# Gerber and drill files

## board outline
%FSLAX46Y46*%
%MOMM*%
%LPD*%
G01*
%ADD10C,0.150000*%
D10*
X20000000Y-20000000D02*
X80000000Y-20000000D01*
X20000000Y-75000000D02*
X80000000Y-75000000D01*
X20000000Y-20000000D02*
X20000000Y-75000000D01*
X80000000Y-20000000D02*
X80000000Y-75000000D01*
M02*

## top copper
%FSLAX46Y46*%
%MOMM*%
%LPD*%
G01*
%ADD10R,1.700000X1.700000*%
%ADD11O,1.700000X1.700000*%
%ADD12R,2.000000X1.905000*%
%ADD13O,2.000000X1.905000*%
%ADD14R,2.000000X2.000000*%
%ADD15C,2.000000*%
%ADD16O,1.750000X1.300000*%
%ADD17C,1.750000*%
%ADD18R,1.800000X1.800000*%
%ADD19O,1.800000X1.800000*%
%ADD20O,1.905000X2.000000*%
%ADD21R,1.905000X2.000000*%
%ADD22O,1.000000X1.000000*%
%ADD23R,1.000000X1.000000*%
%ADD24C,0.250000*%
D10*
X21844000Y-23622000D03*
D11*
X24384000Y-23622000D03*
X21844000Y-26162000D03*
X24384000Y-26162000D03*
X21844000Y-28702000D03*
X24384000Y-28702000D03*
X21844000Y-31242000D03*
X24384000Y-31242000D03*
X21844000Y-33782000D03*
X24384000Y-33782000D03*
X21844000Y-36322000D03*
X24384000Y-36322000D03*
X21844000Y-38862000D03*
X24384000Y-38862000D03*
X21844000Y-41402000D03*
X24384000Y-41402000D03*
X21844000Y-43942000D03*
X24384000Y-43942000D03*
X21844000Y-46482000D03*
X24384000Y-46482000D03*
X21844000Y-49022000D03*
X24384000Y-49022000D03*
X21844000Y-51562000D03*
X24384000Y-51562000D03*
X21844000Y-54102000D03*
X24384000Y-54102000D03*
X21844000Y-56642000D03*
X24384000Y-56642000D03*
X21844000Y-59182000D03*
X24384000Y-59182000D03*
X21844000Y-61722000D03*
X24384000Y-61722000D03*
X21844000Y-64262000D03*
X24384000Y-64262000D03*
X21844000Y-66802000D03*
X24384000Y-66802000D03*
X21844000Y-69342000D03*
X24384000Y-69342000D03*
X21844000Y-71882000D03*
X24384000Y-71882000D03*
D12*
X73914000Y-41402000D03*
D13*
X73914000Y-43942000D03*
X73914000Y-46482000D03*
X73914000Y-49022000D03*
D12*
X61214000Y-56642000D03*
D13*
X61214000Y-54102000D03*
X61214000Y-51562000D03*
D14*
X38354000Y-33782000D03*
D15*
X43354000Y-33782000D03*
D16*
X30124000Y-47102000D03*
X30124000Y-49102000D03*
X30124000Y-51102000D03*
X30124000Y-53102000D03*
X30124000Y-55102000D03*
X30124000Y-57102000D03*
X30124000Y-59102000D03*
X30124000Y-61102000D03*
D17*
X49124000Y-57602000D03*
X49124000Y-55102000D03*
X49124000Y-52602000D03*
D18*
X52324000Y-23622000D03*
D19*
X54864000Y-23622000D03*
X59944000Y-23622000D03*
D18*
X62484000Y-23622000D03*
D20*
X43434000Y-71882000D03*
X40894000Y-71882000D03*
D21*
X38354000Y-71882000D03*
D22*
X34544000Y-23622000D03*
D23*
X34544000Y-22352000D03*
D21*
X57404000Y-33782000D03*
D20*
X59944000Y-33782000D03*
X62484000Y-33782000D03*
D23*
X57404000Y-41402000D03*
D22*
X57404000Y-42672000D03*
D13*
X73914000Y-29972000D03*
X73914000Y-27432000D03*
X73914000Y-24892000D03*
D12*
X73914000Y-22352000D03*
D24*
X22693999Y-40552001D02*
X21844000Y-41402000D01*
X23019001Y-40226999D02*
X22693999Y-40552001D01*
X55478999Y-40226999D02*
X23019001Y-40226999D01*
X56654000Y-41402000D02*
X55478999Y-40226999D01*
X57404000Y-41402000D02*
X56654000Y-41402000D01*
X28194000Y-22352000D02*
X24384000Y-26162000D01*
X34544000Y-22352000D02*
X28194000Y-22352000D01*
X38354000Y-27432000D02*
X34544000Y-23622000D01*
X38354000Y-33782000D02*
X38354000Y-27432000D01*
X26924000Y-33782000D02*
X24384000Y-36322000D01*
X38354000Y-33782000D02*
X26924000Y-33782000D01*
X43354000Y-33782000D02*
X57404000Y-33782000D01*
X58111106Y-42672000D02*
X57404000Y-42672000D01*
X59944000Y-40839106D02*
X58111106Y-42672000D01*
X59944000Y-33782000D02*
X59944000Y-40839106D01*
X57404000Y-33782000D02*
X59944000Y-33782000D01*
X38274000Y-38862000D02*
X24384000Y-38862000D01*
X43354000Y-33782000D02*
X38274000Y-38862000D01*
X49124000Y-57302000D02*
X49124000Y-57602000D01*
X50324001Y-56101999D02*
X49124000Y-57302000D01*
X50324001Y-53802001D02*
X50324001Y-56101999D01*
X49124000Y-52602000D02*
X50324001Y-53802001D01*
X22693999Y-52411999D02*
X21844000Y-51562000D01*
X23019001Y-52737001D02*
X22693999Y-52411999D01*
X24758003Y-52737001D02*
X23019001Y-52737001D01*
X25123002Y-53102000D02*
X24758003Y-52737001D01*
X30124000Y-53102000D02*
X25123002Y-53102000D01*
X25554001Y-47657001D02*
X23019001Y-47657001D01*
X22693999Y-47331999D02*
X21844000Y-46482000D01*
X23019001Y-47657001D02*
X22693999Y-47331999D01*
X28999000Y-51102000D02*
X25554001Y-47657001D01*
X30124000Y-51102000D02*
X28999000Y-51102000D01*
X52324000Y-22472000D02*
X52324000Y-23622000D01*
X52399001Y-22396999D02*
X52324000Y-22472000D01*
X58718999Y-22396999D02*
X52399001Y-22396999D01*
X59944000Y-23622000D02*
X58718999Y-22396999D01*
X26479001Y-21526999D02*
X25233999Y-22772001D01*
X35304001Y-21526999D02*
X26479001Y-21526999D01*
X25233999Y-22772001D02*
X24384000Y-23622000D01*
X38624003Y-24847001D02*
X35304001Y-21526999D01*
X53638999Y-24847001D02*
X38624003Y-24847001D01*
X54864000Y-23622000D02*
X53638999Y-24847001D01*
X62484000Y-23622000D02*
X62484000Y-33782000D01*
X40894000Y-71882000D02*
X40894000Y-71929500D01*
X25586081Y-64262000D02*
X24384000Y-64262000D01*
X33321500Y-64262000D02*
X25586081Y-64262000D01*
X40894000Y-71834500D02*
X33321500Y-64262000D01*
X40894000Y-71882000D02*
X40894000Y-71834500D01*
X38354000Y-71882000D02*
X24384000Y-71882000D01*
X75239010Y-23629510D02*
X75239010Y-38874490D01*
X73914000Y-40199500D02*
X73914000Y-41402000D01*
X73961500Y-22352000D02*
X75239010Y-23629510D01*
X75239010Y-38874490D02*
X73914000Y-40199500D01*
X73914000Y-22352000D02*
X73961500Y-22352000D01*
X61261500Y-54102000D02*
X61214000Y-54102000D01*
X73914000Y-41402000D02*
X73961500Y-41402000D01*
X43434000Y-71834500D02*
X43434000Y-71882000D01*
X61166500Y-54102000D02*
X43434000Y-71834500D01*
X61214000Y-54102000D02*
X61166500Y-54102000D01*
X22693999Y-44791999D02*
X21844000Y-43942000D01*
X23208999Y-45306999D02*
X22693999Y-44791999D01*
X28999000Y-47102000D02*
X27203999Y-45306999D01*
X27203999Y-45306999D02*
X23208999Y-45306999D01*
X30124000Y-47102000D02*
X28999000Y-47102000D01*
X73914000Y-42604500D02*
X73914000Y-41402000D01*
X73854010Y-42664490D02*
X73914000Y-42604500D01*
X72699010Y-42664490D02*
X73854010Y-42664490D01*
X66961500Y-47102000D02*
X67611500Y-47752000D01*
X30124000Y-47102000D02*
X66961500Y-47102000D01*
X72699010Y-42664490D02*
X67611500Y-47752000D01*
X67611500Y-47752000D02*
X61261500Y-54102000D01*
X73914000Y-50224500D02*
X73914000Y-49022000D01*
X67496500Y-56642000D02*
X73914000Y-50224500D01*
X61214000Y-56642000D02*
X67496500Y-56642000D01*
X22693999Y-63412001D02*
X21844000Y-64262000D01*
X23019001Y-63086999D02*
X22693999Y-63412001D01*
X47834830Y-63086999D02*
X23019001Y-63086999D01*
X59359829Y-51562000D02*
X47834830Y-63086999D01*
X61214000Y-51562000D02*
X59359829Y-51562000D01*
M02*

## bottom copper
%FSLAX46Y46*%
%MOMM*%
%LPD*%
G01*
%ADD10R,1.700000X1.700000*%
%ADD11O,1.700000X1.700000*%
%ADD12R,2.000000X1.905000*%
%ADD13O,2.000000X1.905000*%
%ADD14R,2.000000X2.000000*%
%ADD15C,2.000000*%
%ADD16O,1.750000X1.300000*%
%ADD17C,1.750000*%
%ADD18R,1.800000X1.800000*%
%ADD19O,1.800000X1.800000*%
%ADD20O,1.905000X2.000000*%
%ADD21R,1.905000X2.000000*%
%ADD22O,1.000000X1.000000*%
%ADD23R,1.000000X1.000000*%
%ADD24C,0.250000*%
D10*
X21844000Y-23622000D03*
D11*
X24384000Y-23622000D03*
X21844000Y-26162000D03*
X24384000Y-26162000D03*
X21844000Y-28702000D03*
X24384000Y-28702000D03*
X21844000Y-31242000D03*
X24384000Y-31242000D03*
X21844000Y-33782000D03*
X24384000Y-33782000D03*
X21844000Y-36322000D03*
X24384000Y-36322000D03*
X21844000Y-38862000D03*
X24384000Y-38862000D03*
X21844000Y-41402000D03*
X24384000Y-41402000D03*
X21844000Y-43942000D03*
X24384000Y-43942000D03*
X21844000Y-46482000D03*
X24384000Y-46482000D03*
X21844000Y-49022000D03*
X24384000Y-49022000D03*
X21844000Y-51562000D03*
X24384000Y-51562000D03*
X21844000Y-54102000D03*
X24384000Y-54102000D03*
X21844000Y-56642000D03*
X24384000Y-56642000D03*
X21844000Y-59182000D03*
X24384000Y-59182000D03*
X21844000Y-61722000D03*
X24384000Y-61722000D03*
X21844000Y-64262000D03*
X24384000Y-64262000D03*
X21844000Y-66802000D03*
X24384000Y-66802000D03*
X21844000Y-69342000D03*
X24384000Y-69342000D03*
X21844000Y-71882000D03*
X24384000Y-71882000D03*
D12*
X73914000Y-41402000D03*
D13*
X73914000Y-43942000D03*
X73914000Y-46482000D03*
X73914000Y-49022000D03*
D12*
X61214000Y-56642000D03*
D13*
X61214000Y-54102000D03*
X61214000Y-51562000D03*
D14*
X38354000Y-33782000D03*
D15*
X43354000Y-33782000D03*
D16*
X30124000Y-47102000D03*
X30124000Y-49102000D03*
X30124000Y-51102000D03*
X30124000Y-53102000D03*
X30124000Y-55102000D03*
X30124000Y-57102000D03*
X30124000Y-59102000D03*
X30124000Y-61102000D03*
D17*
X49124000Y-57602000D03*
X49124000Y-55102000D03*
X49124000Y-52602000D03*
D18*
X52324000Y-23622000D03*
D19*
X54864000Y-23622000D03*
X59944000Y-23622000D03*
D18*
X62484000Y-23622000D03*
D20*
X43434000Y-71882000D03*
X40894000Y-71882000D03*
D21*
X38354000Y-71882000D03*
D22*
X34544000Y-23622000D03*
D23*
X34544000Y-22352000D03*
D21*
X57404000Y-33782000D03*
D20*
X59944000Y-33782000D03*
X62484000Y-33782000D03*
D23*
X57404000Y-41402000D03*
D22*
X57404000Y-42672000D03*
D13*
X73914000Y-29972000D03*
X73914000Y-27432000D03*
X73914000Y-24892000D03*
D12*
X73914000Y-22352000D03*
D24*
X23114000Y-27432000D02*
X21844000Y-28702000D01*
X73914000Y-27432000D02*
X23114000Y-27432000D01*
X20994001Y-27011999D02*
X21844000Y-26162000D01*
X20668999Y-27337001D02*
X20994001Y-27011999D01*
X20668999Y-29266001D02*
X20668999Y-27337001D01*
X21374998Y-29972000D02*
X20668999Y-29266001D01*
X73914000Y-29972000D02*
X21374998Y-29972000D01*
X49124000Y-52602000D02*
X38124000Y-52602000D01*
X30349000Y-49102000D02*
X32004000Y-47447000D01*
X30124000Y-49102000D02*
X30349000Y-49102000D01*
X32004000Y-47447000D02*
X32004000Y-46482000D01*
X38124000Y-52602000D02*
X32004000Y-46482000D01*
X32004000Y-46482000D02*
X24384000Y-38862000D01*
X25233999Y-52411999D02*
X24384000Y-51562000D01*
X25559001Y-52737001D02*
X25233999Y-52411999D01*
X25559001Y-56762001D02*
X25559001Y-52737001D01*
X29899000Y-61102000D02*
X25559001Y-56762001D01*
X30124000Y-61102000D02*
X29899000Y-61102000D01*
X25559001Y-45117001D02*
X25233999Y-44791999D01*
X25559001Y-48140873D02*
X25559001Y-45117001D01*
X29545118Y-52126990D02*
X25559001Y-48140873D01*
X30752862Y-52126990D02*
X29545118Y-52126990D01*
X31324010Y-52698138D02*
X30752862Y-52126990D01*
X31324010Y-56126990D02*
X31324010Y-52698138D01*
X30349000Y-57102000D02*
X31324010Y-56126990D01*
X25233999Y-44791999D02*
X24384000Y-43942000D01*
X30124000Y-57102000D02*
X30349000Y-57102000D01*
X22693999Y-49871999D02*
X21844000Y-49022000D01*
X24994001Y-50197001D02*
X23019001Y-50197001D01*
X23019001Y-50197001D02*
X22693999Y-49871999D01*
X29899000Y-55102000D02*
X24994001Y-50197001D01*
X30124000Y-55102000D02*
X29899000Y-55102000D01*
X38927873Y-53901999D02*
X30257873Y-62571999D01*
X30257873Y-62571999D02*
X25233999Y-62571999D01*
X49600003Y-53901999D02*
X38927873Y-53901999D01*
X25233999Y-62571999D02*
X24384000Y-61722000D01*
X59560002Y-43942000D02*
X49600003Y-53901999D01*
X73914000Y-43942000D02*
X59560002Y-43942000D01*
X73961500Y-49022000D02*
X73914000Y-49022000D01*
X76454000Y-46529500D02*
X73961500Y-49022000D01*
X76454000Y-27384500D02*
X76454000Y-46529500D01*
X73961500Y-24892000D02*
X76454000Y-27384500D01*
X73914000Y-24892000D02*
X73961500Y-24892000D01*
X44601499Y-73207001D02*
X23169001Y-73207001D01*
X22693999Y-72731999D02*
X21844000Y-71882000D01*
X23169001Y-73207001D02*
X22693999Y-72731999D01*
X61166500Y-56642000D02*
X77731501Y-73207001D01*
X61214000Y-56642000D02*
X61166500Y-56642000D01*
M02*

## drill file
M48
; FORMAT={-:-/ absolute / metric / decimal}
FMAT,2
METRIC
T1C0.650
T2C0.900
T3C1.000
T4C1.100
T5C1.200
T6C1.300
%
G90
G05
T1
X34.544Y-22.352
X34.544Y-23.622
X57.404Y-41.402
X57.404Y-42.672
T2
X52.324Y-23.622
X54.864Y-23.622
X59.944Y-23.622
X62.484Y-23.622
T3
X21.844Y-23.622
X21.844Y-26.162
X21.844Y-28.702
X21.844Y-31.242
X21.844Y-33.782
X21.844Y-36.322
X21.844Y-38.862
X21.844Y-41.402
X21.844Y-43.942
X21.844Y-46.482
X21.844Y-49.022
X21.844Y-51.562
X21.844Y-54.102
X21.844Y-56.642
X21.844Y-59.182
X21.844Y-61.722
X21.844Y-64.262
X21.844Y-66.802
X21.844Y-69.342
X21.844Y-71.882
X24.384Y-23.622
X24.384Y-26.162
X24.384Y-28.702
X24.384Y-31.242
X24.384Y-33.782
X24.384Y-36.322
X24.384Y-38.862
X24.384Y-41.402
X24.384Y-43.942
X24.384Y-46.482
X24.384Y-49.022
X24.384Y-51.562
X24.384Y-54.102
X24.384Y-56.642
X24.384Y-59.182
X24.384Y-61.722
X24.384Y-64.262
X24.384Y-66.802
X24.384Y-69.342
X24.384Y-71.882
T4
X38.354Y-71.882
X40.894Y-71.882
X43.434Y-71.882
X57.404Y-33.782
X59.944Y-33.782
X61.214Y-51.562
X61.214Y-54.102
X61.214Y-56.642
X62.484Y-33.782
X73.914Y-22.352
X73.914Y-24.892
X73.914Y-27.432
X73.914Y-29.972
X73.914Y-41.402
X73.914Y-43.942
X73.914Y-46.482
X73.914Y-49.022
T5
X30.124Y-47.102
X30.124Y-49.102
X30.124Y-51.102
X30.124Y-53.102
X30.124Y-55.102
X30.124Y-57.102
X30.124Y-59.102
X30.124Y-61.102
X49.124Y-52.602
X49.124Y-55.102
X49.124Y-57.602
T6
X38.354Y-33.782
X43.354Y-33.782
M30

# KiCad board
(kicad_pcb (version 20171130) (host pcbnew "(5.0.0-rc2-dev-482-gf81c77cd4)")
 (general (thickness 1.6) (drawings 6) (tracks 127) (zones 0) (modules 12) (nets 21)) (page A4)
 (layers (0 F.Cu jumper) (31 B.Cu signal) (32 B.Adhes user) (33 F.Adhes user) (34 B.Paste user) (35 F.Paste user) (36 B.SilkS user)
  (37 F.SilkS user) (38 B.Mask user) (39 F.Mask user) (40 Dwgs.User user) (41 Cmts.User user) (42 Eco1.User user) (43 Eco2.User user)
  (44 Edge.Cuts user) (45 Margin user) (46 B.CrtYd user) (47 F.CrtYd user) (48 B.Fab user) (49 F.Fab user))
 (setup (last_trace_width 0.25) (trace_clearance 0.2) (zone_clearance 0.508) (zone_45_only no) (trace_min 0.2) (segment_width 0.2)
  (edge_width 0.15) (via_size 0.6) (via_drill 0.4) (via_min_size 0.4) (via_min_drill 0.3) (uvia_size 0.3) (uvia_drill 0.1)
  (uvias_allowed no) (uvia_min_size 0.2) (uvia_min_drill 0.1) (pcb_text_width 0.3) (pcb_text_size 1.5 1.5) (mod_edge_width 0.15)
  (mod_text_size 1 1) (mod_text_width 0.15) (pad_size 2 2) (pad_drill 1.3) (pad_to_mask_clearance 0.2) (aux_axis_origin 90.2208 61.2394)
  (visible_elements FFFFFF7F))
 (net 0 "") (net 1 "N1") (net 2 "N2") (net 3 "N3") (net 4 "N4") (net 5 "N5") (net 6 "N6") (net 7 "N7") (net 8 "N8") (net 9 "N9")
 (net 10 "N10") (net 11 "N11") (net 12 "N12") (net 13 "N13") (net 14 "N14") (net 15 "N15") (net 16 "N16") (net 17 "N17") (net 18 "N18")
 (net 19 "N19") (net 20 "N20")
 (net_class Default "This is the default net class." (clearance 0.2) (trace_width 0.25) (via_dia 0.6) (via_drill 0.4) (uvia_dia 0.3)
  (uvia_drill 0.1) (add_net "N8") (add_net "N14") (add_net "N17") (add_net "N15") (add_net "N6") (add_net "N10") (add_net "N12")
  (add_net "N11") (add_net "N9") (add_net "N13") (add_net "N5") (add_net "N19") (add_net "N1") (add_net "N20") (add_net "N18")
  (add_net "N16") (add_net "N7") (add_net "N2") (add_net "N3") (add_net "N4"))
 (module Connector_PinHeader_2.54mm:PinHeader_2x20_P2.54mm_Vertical (layer F.Cu) (at 21.844 23.622)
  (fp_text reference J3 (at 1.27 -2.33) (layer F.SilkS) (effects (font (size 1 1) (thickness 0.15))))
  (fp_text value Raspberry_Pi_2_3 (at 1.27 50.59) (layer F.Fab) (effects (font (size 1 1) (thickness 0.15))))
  (pad 1 thru_hole rect (at 0 0) (size 1.7 1.7) (drill 1) (layers *.Cu *.Mask))
  (pad 2 thru_hole oval (at 2.54 0) (size 1.7 1.7) (drill 1) (layers *.Cu *.Mask) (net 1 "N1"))
  (pad 3 thru_hole oval (at 0 2.54) (size 1.7 1.7) (drill 1) (layers *.Cu *.Mask) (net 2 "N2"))
  (pad 4 thru_hole oval (at 2.54 2.54) (size 1.7 1.7) (drill 1) (layers *.Cu *.Mask) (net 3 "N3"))
  (pad 5 thru_hole oval (at 0 5.08) (size 1.7 1.7) (drill 1) (layers *.Cu *.Mask) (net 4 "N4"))
  (pad 6 thru_hole oval (at 2.54 5.08) (size 1.7 1.7) (drill 1) (layers *.Cu *.Mask))
  (pad 7 thru_hole oval (at 0 7.62) (size 1.7 1.7) (drill 1) (layers *.Cu *.Mask))
  (pad 8 thru_hole oval (at 2.54 7.62) (size 1.7 1.7) (drill 1) (layers *.Cu *.Mask))
  (pad 9 thru_hole oval (at 0 10.16) (size 1.7 1.7) (drill 1) (layers *.Cu *.Mask))
  (pad 10 thru_hole oval (at 2.54 10.16) (size 1.7 1.7) (drill 1) (layers *.Cu *.Mask))
  (pad 11 thru_hole oval (at 0 12.7) (size 1.7 1.7) (drill 1) (layers *.Cu *.Mask))
  (pad 12 thru_hole oval (at 2.54 12.7) (size 1.7 1.7) (drill 1) (layers *.Cu *.Mask) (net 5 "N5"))
  (pad 13 thru_hole oval (at 0 15.24) (size 1.7 1.7) (drill 1) (layers *.Cu *.Mask))
  (pad 14 thru_hole oval (at 2.54 15.24) (size 1.7 1.7) (drill 1) (layers *.Cu *.Mask) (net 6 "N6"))
  (pad 15 thru_hole oval (at 0 17.78) (size 1.7 1.7) (drill 1) (layers *.Cu *.Mask) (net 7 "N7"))
  (pad 16 thru_hole oval (at 2.54 17.78) (size 1.7 1.7) (drill 1) (layers *.Cu *.Mask))
  (pad 17 thru_hole oval (at 0 20.32) (size 1.7 1.7) (drill 1) (layers *.Cu *.Mask) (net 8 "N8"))
  (pad 18 thru_hole oval (at 2.54 20.32) (size 1.7 1.7) (drill 1) (layers *.Cu *.Mask) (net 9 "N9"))
  (pad 19 thru_hole oval (at 0 22.86) (size 1.7 1.7) (drill 1) (layers *.Cu *.Mask) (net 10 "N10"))
  (pad 20 thru_hole oval (at 2.54 22.86) (size 1.7 1.7) (drill 1) (layers *.Cu *.Mask))
  (pad 21 thru_hole oval (at 0 25.4) (size 1.7 1.7) (drill 1) (layers *.Cu *.Mask) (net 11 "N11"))
  (pad 22 thru_hole oval (at 2.54 25.4) (size 1.7 1.7) (drill 1) (layers *.Cu *.Mask))
  (pad 23 thru_hole oval (at 0 27.94) (size 1.7 1.7) (drill 1) (layers *.Cu *.Mask) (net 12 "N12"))
  (pad 24 thru_hole oval (at 2.54 27.94) (size 1.7 1.7) (drill 1) (layers *.Cu *.Mask) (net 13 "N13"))
  (pad 25 thru_hole oval (at 0 30.48) (size 1.7 1.7) (drill 1) (layers *.Cu *.Mask))
  (pad 26 thru_hole oval (at 2.54 30.48) (size 1.7 1.7) (drill 1) (layers *.Cu *.Mask))
  (pad 27 thru_hole oval (at 0 33.02) (size 1.7 1.7) (drill 1) (layers *.Cu *.Mask))
  (pad 28 thru_hole oval (at 2.54 33.02) (size 1.7 1.7) (drill 1) (layers *.Cu *.Mask))
  (pad 29 thru_hole oval (at 0 35.56) (size 1.7 1.7) (drill 1) (layers *.Cu *.Mask))
  (pad 30 thru_hole oval (at 2.54 35.56) (size 1.7 1.7) (drill 1) (layers *.Cu *.Mask))
  (pad 31 thru_hole oval (at 0 38.1) (size 1.7 1.7) (drill 1) (layers *.Cu *.Mask))
  (pad 32 thru_hole oval (at 2.54 38.1) (size 1.7 1.7) (drill 1) (layers *.Cu *.Mask) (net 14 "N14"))
  (pad 33 thru_hole oval (at 0 40.64) (size 1.7 1.7) (drill 1) (layers *.Cu *.Mask) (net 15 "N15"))
  (pad 34 thru_hole oval (at 2.54 40.64) (size 1.7 1.7) (drill 1) (layers *.Cu *.Mask) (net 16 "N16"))
  (pad 35 thru_hole oval (at 0 43.18) (size 1.7 1.7) (drill 1) (layers *.Cu *.Mask))
  (pad 36 thru_hole oval (at 2.54 43.18) (size 1.7 1.7) (drill 1) (layers *.Cu *.Mask))
  (pad 37 thru_hole oval (at 0 45.72) (size 1.7 1.7) (drill 1) (layers *.Cu *.Mask))
  (pad 38 thru_hole oval (at 2.54 45.72) (size 1.7 1.7) (drill 1) (layers *.Cu *.Mask))
  (pad 39 thru_hole oval (at 0 48.26) (size 1.7 1.7) (drill 1) (layers *.Cu *.Mask) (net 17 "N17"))
  (pad 40 thru_hole oval (at 2.54 48.26) (size 1.7 1.7) (drill 1) (layers *.Cu *.Mask) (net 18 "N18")))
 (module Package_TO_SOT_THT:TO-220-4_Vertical (layer F.Cu) (at 73.914 41.402 270)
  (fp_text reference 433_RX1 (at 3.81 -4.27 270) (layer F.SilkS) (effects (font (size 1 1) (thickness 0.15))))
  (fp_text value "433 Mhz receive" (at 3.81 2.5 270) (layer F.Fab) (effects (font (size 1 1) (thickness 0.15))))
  (pad 1 thru_hole rect (at 0 0 270) (size 1.905 2) (drill 1.1) (layers *.Cu *.Mask) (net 8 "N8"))
  (pad 2 thru_hole oval (at 2.54 0 270) (size 1.905 2) (drill 1.1) (layers *.Cu *.Mask) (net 14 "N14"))
  (pad 3 thru_hole oval (at 5.08 0 270) (size 1.905 2) (drill 1.1) (layers *.Cu *.Mask))
  (pad 4 thru_hole oval (at 7.62 0 270) (size 1.905 2) (drill 1.1) (layers *.Cu *.Mask) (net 17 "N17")))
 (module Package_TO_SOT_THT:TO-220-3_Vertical (layer F.Cu) (at 61.214 56.642 90)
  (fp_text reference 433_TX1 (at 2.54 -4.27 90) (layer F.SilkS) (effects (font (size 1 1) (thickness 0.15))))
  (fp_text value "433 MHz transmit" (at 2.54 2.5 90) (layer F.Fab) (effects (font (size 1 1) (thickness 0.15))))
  (pad 1 thru_hole rect (at 0 0 90) (size 1.905 2) (drill 1.1) (layers *.Cu *.Mask) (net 17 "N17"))
  (pad 2 thru_hole oval (at 2.54 0 90) (size 1.905 2) (drill 1.1) (layers *.Cu *.Mask) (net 8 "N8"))
  (pad 3 thru_hole oval (at 5.08 0 90) (size 1.905 2) (drill 1.1) (layers *.Cu *.Mask) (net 15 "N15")))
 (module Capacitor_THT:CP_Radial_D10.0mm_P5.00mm (layer F.Cu) (at 38.354 33.782)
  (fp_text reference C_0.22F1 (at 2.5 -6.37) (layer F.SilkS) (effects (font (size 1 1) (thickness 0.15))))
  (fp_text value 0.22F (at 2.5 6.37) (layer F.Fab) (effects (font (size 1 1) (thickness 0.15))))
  (pad 1 thru_hole rect (at 0 0) (size 2 2) (drill 1.3) (layers *.Cu *.Mask) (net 5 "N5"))
  (pad 2 thru_hole circle (at 5 0) (size 2 2) (drill 1.3) (layers *.Cu *.Mask) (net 6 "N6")))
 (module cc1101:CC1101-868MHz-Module (layer F.Cu) (at 39.624 54.102)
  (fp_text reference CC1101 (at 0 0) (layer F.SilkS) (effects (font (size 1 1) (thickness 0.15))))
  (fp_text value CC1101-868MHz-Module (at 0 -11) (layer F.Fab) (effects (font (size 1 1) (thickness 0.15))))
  (pad 1 thru_hole oval (at -9.5 -7) (size 1.75 1.3) (drill 1.2) (layers *.Cu *.Mask) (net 8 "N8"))
  (pad 2 thru_hole oval (at -9.5 -5) (size 1.75 1.3) (drill 1.2) (layers *.Cu *.Mask) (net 6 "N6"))
  (pad 3 thru_hole oval (at -9.5 -3) (size 1.75 1.3) (drill 1.2) (layers *.Cu *.Mask) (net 10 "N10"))
  (pad 4 thru_hole oval (at -9.5 -1) (size 1.75 1.3) (drill 1.2) (layers *.Cu *.Mask) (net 12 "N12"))
  (pad 5 thru_hole oval (at -9.5 1) (size 1.75 1.3) (drill 1.2) (layers *.Cu *.Mask) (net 11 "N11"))
  (pad 6 thru_hole oval (at -9.5 3) (size 1.75 1.3) (drill 1.2) (layers *.Cu *.Mask) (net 9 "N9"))
  (pad 7 thru_hole oval (at -9.5 5) (size 1.75 1.3) (drill 1.2) (layers *.Cu *.Mask))
  (pad 8 thru_hole oval (at -9.5 7) (size 1.75 1.3) (drill 1.2) (layers *.Cu *.Mask) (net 13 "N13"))
  (pad 9 thru_hole circle (at 9.5 3.5) (size 1.75 1.75) (drill 1.2) (layers *.Cu *.Mask) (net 6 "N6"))
  (pad 10 thru_hole circle (at 9.5 1) (size 1.75 1.75) (drill 1.2) (layers *.Cu *.Mask))
  (pad 11 thru_hole circle (at 9.5 -1.5) (size 1.75 1.75) (drill 1.2) (layers *.Cu *.Mask) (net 6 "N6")))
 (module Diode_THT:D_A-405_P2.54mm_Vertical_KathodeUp (layer F.Cu) (at 52.324 23.622)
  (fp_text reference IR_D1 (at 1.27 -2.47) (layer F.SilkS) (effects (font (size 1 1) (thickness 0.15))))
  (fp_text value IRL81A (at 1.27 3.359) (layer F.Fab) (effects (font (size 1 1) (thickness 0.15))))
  (pad 1 thru_hole rect (at 0 0) (size 1.8 1.8) (drill 0.9) (layers *.Cu *.Mask) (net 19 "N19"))
  (pad 2 thru_hole oval (at 2.54 0) (size 1.8 1.8) (drill 0.9) (layers *.Cu *.Mask) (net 1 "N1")))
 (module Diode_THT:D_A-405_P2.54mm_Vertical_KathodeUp (layer F.Cu) (at 62.484 23.622 180)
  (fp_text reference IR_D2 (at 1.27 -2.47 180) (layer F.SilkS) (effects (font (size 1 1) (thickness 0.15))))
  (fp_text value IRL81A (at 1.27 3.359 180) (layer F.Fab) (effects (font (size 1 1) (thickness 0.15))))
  (pad 2 thru_hole oval (at 2.54 0 180) (size 1.8 1.8) (drill 0.9) (layers *.Cu *.Mask) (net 19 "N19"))
  (pad 1 thru_hole rect (at 0 0 180) (size 1.8 1.8) (drill 0.9) (layers *.Cu *.Mask) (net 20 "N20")))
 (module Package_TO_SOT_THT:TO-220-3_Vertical (layer F.Cu) (at 38.354 71.882)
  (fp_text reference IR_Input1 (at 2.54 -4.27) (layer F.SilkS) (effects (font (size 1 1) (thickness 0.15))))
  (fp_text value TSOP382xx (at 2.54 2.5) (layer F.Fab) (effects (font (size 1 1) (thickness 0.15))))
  (pad 3 thru_hole oval (at 5.08 0) (size 1.905 2) (drill 1.1) (layers *.Cu *.Mask) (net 8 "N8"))
  (pad 2 thru_hole oval (at 2.54 0) (size 1.905 2) (drill 1.1) (layers *.Cu *.Mask) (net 16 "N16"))
  (pad 1 thru_hole rect (at 0 0) (size 1.905 2) (drill 1.1) (layers *.Cu *.Mask) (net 18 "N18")))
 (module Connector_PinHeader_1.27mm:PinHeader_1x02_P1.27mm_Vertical (layer F.Cu) (at 34.544 22.352)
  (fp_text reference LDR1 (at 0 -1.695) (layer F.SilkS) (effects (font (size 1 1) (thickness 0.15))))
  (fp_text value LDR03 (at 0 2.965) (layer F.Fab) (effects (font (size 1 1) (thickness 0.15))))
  (pad 2 thru_hole oval (at 0 1.27) (size 1 1) (drill 0.65) (layers *.Cu *.Mask) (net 5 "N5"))
  (pad 1 thru_hole rect (at 0 0) (size 1 1) (drill 0.65) (layers *.Cu *.Mask) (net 3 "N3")))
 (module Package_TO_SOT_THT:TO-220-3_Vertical (layer F.Cu) (at 57.404 33.782)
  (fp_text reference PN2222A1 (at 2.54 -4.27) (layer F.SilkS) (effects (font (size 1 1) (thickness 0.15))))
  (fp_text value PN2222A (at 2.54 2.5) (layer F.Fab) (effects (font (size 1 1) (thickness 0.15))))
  (pad 1 thru_hole rect (at 0 0) (size 1.905 2) (drill 1.1) (layers *.Cu *.Mask) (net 6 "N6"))
  (pad 2 thru_hole oval (at 2.54 0) (size 1.905 2) (drill 1.1) (layers *.Cu *.Mask) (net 6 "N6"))
  (pad 3 thru_hole oval (at 5.08 0) (size 1.905 2) (drill 1.1) (layers *.Cu *.Mask) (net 20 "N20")))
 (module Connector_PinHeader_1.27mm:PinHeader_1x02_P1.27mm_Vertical (layer F.Cu) (at 57.404 41.402)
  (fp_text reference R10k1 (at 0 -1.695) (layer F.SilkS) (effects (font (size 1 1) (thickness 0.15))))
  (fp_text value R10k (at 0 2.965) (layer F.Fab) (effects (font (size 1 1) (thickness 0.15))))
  (pad 1 thru_hole rect (at 0 0) (size 1 1) (drill 0.65) (layers *.Cu *.Mask) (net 7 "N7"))
  (pad 2 thru_hole oval (at 0 1.27) (size 1 1) (drill 0.65) (layers *.Cu *.Mask) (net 6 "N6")))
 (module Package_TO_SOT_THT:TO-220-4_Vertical (layer F.Cu) (at 73.914 22.352 270)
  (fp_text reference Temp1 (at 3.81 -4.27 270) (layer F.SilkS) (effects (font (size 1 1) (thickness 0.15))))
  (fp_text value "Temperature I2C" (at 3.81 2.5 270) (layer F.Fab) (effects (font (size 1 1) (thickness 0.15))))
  (pad 4 thru_hole oval (at 7.62 0 270) (size 1.905 2) (drill 1.1) (layers *.Cu *.Mask) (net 2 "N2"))
  (pad 3 thru_hole oval (at 5.08 0 270) (size 1.905 2) (drill 1.1) (layers *.Cu *.Mask) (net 4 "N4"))
  (pad 2 thru_hole oval (at 2.54 0 270) (size 1.905 2) (drill 1.1) (layers *.Cu *.Mask) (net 17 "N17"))
  (pad 1 thru_hole rect (at 0 0 270) (size 1.905 2) (drill 1.1) (layers *.Cu *.Mask) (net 8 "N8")))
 (gr_line (start 20 20) (end 80 20) (angle 90) (layer Edge.Cuts) (width 0.15))
 (gr_line (start 20 75) (end 80 75) (angle 90) (layer Edge.Cuts) (width 0.15))
 (gr_line (start 20 20) (end 20 75) (angle 90) (layer Edge.Cuts) (width 0.15))
 (gr_line (start 80 20) (end 80 75) (angle 90) (layer Edge.Cuts) (width 0.15))
 (segment (start 22.693999 40.552001) (end 21.844 41.402) (width 0.25) (layer F.Cu) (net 7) (status 30))
 (segment (start 23.019001 40.226999) (end 22.693999 40.552001) (width 0.25) (layer F.Cu) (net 7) (status 20))
 (segment (start 55.478999 40.226999) (end 23.019001 40.226999) (width 0.25) (layer F.Cu) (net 7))
 (segment (start 56.654 41.402) (end 55.478999 40.226999) (width 0.25) (layer F.Cu) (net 7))
 (segment (start 57.404 41.402) (end 56.654 41.402) (width 0.25) (layer F.Cu) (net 7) (status 10))
 (segment (start 23.114 27.432) (end 21.844 28.702) (width 0.25) (layer B.Cu) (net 4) (status 20))
 (segment (start 73.914 27.432) (end 23.114 27.432) (width 0.25) (layer B.Cu) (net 4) (status 10))
 (segment (start 20.994001 27.011999) (end 21.844 26.162) (width 0.25) (layer B.Cu) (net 2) (status 30))
 (segment (start 20.668999 27.337001) (end 20.994001 27.011999) (width 0.25) (layer B.Cu) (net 2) (status 20))
 (segment (start 20.668999 29.266001) (end 20.668999 27.337001) (width 0.25) (layer B.Cu) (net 2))
 (segment (start 21.374998 29.972) (end 20.668999 29.266001) (width 0.25) (layer B.Cu) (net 2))
 (segment (start 73.914 29.972) (end 21.374998 29.972) (width 0.25) (layer B.Cu) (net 2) (status 10))
 (segment (start 28.194 22.352) (end 24.384 26.162) (width 0.25) (layer F.Cu) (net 3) (status 20))
 (segment (start 34.544 22.352) (end 28.194 22.352) (width 0.25) (layer F.Cu) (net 3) (status 10))
 (segment (start 38.354 27.432) (end 34.544 23.622) (width 0.25) (layer F.Cu) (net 5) (status 20))
 (segment (start 38.354 33.782) (end 38.354 27.432) (width 0.25) (layer F.Cu) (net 5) (status 10))
 (segment (start 26.924 33.782) (end 24.384 36.322) (width 0.25) (layer F.Cu) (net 5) (status 20))
 (segment (start 38.354 33.782) (end 26.924 33.782) (width 0.25) (layer F.Cu) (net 5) (status 10))
 (segment (start 43.354 33.782) (end 57.404 33.782) (width 0.25) (layer F.Cu) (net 6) (status 30))
 (segment (start 58.111106 42.672) (end 57.404 42.672) (width 0.25) (layer F.Cu) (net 6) (status 20))
 (segment (start 59.944 40.839106) (end 58.111106 42.672) (width 0.25) (layer F.Cu) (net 6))
 (segment (start 59.944 33.782) (end 59.944 40.839106) (width 0.25) (layer F.Cu) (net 6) (status 10))
 (segment (start 57.404 33.782) (end 59.944 33.782) (width 0.25) (layer F.Cu) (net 6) (status 30))
 (segment (start 38.274 38.862) (end 24.384 38.862) (width 0.25) (layer F.Cu) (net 6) (status 20))
 (segment (start 43.354 33.782) (end 38.274 38.862) (width 0.25) (layer F.Cu) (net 6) (status 10))
 (segment (start 49.124 52.602) (end 38.124 52.602) (width 0.25) (layer B.Cu) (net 6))
 (segment (start 30.349 49.102) (end 32.004 47.447) (width 0.25) (layer B.Cu) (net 6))
 (segment (start 30.124 49.102) (end 30.349 49.102) (width 0.25) (layer B.Cu) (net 6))
 (segment (start 32.004 47.447) (end 32.004 46.482) (width 0.25) (layer B.Cu) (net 6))
 (segment (start 38.124 52.602) (end 32.004 46.482) (width 0.25) (layer B.Cu) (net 6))
 (segment (start 32.004 46.482) (end 24.384 38.862) (width 0.25) (layer B.Cu) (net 6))
 (segment (start 49.124 57.302) (end 49.124 57.602) (width 0.25) (layer F.Cu) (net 6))
 (segment (start 50.324001 56.101999) (end 49.124 57.302) (width 0.25) (layer F.Cu) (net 6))
 (segment (start 50.324001 53.802001) (end 50.324001 56.101999) (width 0.25) (layer F.Cu) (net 6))
 (segment (start 49.124 52.602) (end 50.324001 53.802001) (width 0.25) (layer F.Cu) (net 6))
 (segment (start 25.233999 52.411999) (end 24.384 51.562) (width 0.25) (layer B.Cu) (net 13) (status 30))
 (segment (start 25.559001 52.737001) (end 25.233999 52.411999) (width 0.25) (layer B.Cu) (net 13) (status 20))
 (segment (start 25.559001 56.762001) (end 25.559001 52.737001) (width 0.25) (layer B.Cu) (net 13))
 (segment (start 29.899 61.102) (end 25.559001 56.762001) (width 0.25) (layer B.Cu) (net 13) (status 10))
 (segment (start 30.124 61.102) (end 29.899 61.102) (width 0.25) (layer B.Cu) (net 13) (status 30))
 (segment (start 25.559001 45.117001) (end 25.233999 44.791999) (width 0.25) (layer B.Cu) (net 9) (status 20))
 (segment (start 25.559001 48.140873) (end 25.559001 45.117001) (width 0.25) (layer B.Cu) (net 9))
 (segment (start 29.545118 52.12699) (end 25.559001 48.140873) (width 0.25) (layer B.Cu) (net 9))
 (segment (start 30.752862 52.12699) (end 29.545118 52.12699) (width 0.25) (layer B.Cu) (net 9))
 (segment (start 31.32401 52.698138) (end 30.752862 52.12699) (width 0.25) (layer B.Cu) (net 9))
 (segment (start 31.32401 56.12699) (end 31.32401 52.698138) (width 0.25) (layer B.Cu) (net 9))
 (segment (start 30.349 57.102) (end 31.32401 56.12699) (width 0.25) (layer B.Cu) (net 9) (status 10))
 (segment (start 25.233999 44.791999) (end 24.384 43.942) (width 0.25) (layer B.Cu) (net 9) (status 30))
 (segment (start 30.124 57.102) (end 30.349 57.102) (width 0.25) (layer B.Cu) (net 9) (status 30))
 (segment (start 22.693999 49.871999) (end 21.844 49.022) (width 0.25) (layer B.Cu) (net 11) (status 30))
 (segment (start 24.994001 50.197001) (end 23.019001 50.197001) (width 0.25) (layer B.Cu) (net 11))
 (segment (start 23.019001 50.197001) (end 22.693999 49.871999) (width 0.25) (layer B.Cu) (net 11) (status 20))
 (segment (start 29.899 55.102) (end 24.994001 50.197001) (width 0.25) (layer B.Cu) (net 11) (status 10))
 (segment (start 30.124 55.102) (end 29.899 55.102) (width 0.25) (layer B.Cu) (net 11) (status 30))
 (segment (start 22.693999 52.411999) (end 21.844 51.562) (width 0.25) (layer F.Cu) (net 12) (status 30))
 (segment (start 23.019001 52.737001) (end 22.693999 52.411999) (width 0.25) (layer F.Cu) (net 12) (status 20))
 (segment (start 24.758003 52.737001) (end 23.019001 52.737001) (width 0.25) (layer F.Cu) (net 12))
 (segment (start 25.123002 53.102) (end 24.758003 52.737001) (width 0.25) (layer F.Cu) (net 12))
 (segment (start 30.124 53.102) (end 25.123002 53.102) (width 0.25) (layer F.Cu) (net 12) (status 10))
 (segment (start 25.554001 47.657001) (end 23.019001 47.657001) (width 0.25) (layer F.Cu) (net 10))
 (segment (start 22.693999 47.331999) (end 21.844 46.482) (width 0.25) (layer F.Cu) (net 10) (status 30))
 (segment (start 23.019001 47.657001) (end 22.693999 47.331999) (width 0.25) (layer F.Cu) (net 10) (status 20))
 (segment (start 28.999 51.102) (end 25.554001 47.657001) (width 0.25) (layer F.Cu) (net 10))
 (segment (start 30.124 51.102) (end 28.999 51.102) (width 0.25) (layer F.Cu) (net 10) (status 10))
 (segment (start 52.324 22.472) (end 52.324 23.622) (width 0.25) (layer F.Cu) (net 19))
 (segment (start 52.399001 22.396999) (end 52.324 22.472) (width 0.25) (layer F.Cu) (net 19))
 (segment (start 58.718999 22.396999) (end 52.399001 22.396999) (width 0.25) (layer F.Cu) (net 19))
 (segment (start 59.944 23.622) (end 58.718999 22.396999) (width 0.25) (layer F.Cu) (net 19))
 (segment (start 26.479001 21.526999) (end 25.233999 22.772001) (width 0.25) (layer F.Cu) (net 1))
 (segment (start 35.304001 21.526999) (end 26.479001 21.526999) (width 0.25) (layer F.Cu) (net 1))
 (segment (start 25.233999 22.772001) (end 24.384 23.622) (width 0.25) (layer F.Cu) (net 1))
 (segment (start 38.624003 24.847001) (end 35.304001 21.526999) (width 0.25) (layer F.Cu) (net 1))
 (segment (start 53.638999 24.847001) (end 38.624003 24.847001) (width 0.25) (layer F.Cu) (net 1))
 (segment (start 54.864 23.622) (end 53.638999 24.847001) (width 0.25) (layer F.Cu) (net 1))
 (segment (start 62.484 23.622) (end 62.484 33.782) (width 0.25) (layer F.Cu) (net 20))
 (segment (start 40.894 71.882) (end 40.894 71.9295) (width 0.25) (layer F.Cu) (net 16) (status 30))
 (segment (start 25.586081 64.262) (end 24.384 64.262) (width 0.25) (layer F.Cu) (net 16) (status 20))
 (segment (start 33.3215 64.262) (end 25.586081 64.262) (width 0.25) (layer F.Cu) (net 16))
 (segment (start 40.894 71.8345) (end 33.3215 64.262) (width 0.25) (layer F.Cu) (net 16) (status 10))
 (segment (start 40.894 71.882) (end 40.894 71.8345) (width 0.25) (layer F.Cu) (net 16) (status 30))
 (segment (start 38.354 71.882) (end 24.384 71.882) (width 0.25) (layer F.Cu) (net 18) (status 30))
 (segment (start 75.23901 23.62951) (end 75.23901 38.87449) (width 0.25) (layer F.Cu) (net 8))
 (segment (start 73.914 40.1995) (end 73.914 41.402) (width 0.25) (layer F.Cu) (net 8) (status 20))
 (segment (start 73.9615 22.352) (end 75.23901 23.62951) (width 0.25) (layer F.Cu) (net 8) (status 10))
 (segment (start 75.23901 38.87449) (end 73.914 40.1995) (width 0.25) (layer F.Cu) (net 8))
 (segment (start 73.914 22.352) (end 73.9615 22.352) (width 0.25) (layer F.Cu) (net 8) (status 30))
 (segment (start 61.2615 54.102) (end 61.214 54.102) (width 0.25) (layer F.Cu) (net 8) (status 30))
 (segment (start 73.914 41.402) (end 73.9615 41.402) (width 0.25) (layer F.Cu) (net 8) (status 30))
 (segment (start 43.434 71.8345) (end 43.434 71.882) (width 0.25) (layer F.Cu) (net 8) (status 30))
 (segment (start 61.1665 54.102) (end 43.434 71.8345) (width 0.25) (layer F.Cu) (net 8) (status 30))
 (segment (start 61.214 54.102) (end 61.1665 54.102) (width 0.25) (layer F.Cu) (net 8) (status 30))
 (segment (start 22.693999 44.791999) (end 21.844 43.942) (width 0.25) (layer F.Cu) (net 8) (status 30))
 (segment (start 23.208999 45.306999) (end 22.693999 44.791999) (width 0.25) (layer F.Cu) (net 8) (status 20))
 (segment (start 28.999 47.102) (end 27.203999 45.306999) (width 0.25) (layer F.Cu) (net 8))
 (segment (start 27.203999 45.306999) (end 23.208999 45.306999) (width 0.25) (layer F.Cu) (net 8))
 (segment (start 30.124 47.102) (end 28.999 47.102) (width 0.25) (layer F.Cu) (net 8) (status 10))
 (segment (start 73.914 42.6045) (end 73.914 41.402) (width 0.25) (layer F.Cu) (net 8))
 (segment (start 73.85401 42.66449) (end 73.914 42.6045) (width 0.25) (layer F.Cu) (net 8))
 (segment (start 72.69901 42.66449) (end 73.85401 42.66449) (width 0.25) (layer F.Cu) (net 8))
 (segment (start 66.9615 47.102) (end 67.6115 47.752) (width 0.25) (layer F.Cu) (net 8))
 (segment (start 30.124 47.102) (end 66.9615 47.102) (width 0.25) (layer F.Cu) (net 8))
 (segment (start 72.69901 42.66449) (end 67.6115 47.752) (width 0.25) (layer F.Cu) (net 8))
 (segment (start 67.6115 47.752) (end 61.2615 54.102) (width 0.25) (layer F.Cu) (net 8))
 (segment (start 38.927873 53.901999) (end 30.257873 62.571999) (width 0.25) (layer B.Cu) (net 14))
 (segment (start 30.257873 62.571999) (end 25.233999 62.571999) (width 0.25) (layer B.Cu) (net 14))
 (segment (start 49.600003 53.901999) (end 38.927873 53.901999) (width 0.25) (layer B.Cu) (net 14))
 (segment (start 25.233999 62.571999) (end 24.384 61.722) (width 0.25) (layer B.Cu) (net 14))
 (segment (start 59.560002 43.942) (end 49.600003 53.901999) (width 0.25) (layer B.Cu) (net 14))
 (segment (start 73.914 43.942) (end 59.560002 43.942) (width 0.25) (layer B.Cu) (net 14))
 (segment (start 73.9615 49.022) (end 73.914 49.022) (width 0.25) (layer B.Cu) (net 17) (status 30))
 (segment (start 76.454 46.5295) (end 73.9615 49.022) (width 0.25) (layer B.Cu) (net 17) (status 20))
 (segment (start 76.454 27.3845) (end 76.454 46.5295) (width 0.25) (layer B.Cu) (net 17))
 (segment (start 73.9615 24.892) (end 76.454 27.3845) (width 0.25) (layer B.Cu) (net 17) (status 10))
 (segment (start 73.914 24.892) (end 73.9615 24.892) (width 0.25) (layer B.Cu) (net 17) (status 30))
 (segment (start 73.914 50.2245) (end 73.914 49.022) (width 0.25) (layer F.Cu) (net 17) (status 20))
 (segment (start 67.4965 56.642) (end 73.914 50.2245) (width 0.25) (layer F.Cu) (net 17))
 (segment (start 61.214 56.642) (end 67.4965 56.642) (width 0.25) (layer F.Cu) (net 17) (status 10))
 (segment (start 44.601499 73.207001) (end 23.169001 73.207001) (width 0.25) (layer B.Cu) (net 17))
 (segment (start 22.693999 72.731999) (end 21.844 71.882) (width 0.25) (layer B.Cu) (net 17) (status 30))
 (segment (start 23.169001 73.207001) (end 22.693999 72.731999) (width 0.25) (layer B.Cu) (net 17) (status 20))
 (segment (start 61.1665 56.642) (end 77.731501 73.207001) (width 0.25) (layer B.Cu) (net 17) (status 10))
 (segment (start 61.214 56.642) (end 61.1665 56.642) (width 0.25) (layer B.Cu) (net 17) (status 30))
 (segment (start 22.693999 63.412001) (end 21.844 64.262) (width 0.25) (layer F.Cu) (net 15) (status 30))
 (segment (start 23.019001 63.086999) (end 22.693999 63.412001) (width 0.25) (layer F.Cu) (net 15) (status 20))
 (segment (start 47.83483 63.086999) (end 23.019001 63.086999) (width 0.25) (layer F.Cu) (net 15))
 (segment (start 59.359829 51.562) (end 47.83483 63.086999) (width 0.25) (layer F.Cu) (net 15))
 (segment (start 61.214 51.562) (end 59.359829 51.562) (width 0.25) (layer F.Cu) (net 15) (status 10)))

